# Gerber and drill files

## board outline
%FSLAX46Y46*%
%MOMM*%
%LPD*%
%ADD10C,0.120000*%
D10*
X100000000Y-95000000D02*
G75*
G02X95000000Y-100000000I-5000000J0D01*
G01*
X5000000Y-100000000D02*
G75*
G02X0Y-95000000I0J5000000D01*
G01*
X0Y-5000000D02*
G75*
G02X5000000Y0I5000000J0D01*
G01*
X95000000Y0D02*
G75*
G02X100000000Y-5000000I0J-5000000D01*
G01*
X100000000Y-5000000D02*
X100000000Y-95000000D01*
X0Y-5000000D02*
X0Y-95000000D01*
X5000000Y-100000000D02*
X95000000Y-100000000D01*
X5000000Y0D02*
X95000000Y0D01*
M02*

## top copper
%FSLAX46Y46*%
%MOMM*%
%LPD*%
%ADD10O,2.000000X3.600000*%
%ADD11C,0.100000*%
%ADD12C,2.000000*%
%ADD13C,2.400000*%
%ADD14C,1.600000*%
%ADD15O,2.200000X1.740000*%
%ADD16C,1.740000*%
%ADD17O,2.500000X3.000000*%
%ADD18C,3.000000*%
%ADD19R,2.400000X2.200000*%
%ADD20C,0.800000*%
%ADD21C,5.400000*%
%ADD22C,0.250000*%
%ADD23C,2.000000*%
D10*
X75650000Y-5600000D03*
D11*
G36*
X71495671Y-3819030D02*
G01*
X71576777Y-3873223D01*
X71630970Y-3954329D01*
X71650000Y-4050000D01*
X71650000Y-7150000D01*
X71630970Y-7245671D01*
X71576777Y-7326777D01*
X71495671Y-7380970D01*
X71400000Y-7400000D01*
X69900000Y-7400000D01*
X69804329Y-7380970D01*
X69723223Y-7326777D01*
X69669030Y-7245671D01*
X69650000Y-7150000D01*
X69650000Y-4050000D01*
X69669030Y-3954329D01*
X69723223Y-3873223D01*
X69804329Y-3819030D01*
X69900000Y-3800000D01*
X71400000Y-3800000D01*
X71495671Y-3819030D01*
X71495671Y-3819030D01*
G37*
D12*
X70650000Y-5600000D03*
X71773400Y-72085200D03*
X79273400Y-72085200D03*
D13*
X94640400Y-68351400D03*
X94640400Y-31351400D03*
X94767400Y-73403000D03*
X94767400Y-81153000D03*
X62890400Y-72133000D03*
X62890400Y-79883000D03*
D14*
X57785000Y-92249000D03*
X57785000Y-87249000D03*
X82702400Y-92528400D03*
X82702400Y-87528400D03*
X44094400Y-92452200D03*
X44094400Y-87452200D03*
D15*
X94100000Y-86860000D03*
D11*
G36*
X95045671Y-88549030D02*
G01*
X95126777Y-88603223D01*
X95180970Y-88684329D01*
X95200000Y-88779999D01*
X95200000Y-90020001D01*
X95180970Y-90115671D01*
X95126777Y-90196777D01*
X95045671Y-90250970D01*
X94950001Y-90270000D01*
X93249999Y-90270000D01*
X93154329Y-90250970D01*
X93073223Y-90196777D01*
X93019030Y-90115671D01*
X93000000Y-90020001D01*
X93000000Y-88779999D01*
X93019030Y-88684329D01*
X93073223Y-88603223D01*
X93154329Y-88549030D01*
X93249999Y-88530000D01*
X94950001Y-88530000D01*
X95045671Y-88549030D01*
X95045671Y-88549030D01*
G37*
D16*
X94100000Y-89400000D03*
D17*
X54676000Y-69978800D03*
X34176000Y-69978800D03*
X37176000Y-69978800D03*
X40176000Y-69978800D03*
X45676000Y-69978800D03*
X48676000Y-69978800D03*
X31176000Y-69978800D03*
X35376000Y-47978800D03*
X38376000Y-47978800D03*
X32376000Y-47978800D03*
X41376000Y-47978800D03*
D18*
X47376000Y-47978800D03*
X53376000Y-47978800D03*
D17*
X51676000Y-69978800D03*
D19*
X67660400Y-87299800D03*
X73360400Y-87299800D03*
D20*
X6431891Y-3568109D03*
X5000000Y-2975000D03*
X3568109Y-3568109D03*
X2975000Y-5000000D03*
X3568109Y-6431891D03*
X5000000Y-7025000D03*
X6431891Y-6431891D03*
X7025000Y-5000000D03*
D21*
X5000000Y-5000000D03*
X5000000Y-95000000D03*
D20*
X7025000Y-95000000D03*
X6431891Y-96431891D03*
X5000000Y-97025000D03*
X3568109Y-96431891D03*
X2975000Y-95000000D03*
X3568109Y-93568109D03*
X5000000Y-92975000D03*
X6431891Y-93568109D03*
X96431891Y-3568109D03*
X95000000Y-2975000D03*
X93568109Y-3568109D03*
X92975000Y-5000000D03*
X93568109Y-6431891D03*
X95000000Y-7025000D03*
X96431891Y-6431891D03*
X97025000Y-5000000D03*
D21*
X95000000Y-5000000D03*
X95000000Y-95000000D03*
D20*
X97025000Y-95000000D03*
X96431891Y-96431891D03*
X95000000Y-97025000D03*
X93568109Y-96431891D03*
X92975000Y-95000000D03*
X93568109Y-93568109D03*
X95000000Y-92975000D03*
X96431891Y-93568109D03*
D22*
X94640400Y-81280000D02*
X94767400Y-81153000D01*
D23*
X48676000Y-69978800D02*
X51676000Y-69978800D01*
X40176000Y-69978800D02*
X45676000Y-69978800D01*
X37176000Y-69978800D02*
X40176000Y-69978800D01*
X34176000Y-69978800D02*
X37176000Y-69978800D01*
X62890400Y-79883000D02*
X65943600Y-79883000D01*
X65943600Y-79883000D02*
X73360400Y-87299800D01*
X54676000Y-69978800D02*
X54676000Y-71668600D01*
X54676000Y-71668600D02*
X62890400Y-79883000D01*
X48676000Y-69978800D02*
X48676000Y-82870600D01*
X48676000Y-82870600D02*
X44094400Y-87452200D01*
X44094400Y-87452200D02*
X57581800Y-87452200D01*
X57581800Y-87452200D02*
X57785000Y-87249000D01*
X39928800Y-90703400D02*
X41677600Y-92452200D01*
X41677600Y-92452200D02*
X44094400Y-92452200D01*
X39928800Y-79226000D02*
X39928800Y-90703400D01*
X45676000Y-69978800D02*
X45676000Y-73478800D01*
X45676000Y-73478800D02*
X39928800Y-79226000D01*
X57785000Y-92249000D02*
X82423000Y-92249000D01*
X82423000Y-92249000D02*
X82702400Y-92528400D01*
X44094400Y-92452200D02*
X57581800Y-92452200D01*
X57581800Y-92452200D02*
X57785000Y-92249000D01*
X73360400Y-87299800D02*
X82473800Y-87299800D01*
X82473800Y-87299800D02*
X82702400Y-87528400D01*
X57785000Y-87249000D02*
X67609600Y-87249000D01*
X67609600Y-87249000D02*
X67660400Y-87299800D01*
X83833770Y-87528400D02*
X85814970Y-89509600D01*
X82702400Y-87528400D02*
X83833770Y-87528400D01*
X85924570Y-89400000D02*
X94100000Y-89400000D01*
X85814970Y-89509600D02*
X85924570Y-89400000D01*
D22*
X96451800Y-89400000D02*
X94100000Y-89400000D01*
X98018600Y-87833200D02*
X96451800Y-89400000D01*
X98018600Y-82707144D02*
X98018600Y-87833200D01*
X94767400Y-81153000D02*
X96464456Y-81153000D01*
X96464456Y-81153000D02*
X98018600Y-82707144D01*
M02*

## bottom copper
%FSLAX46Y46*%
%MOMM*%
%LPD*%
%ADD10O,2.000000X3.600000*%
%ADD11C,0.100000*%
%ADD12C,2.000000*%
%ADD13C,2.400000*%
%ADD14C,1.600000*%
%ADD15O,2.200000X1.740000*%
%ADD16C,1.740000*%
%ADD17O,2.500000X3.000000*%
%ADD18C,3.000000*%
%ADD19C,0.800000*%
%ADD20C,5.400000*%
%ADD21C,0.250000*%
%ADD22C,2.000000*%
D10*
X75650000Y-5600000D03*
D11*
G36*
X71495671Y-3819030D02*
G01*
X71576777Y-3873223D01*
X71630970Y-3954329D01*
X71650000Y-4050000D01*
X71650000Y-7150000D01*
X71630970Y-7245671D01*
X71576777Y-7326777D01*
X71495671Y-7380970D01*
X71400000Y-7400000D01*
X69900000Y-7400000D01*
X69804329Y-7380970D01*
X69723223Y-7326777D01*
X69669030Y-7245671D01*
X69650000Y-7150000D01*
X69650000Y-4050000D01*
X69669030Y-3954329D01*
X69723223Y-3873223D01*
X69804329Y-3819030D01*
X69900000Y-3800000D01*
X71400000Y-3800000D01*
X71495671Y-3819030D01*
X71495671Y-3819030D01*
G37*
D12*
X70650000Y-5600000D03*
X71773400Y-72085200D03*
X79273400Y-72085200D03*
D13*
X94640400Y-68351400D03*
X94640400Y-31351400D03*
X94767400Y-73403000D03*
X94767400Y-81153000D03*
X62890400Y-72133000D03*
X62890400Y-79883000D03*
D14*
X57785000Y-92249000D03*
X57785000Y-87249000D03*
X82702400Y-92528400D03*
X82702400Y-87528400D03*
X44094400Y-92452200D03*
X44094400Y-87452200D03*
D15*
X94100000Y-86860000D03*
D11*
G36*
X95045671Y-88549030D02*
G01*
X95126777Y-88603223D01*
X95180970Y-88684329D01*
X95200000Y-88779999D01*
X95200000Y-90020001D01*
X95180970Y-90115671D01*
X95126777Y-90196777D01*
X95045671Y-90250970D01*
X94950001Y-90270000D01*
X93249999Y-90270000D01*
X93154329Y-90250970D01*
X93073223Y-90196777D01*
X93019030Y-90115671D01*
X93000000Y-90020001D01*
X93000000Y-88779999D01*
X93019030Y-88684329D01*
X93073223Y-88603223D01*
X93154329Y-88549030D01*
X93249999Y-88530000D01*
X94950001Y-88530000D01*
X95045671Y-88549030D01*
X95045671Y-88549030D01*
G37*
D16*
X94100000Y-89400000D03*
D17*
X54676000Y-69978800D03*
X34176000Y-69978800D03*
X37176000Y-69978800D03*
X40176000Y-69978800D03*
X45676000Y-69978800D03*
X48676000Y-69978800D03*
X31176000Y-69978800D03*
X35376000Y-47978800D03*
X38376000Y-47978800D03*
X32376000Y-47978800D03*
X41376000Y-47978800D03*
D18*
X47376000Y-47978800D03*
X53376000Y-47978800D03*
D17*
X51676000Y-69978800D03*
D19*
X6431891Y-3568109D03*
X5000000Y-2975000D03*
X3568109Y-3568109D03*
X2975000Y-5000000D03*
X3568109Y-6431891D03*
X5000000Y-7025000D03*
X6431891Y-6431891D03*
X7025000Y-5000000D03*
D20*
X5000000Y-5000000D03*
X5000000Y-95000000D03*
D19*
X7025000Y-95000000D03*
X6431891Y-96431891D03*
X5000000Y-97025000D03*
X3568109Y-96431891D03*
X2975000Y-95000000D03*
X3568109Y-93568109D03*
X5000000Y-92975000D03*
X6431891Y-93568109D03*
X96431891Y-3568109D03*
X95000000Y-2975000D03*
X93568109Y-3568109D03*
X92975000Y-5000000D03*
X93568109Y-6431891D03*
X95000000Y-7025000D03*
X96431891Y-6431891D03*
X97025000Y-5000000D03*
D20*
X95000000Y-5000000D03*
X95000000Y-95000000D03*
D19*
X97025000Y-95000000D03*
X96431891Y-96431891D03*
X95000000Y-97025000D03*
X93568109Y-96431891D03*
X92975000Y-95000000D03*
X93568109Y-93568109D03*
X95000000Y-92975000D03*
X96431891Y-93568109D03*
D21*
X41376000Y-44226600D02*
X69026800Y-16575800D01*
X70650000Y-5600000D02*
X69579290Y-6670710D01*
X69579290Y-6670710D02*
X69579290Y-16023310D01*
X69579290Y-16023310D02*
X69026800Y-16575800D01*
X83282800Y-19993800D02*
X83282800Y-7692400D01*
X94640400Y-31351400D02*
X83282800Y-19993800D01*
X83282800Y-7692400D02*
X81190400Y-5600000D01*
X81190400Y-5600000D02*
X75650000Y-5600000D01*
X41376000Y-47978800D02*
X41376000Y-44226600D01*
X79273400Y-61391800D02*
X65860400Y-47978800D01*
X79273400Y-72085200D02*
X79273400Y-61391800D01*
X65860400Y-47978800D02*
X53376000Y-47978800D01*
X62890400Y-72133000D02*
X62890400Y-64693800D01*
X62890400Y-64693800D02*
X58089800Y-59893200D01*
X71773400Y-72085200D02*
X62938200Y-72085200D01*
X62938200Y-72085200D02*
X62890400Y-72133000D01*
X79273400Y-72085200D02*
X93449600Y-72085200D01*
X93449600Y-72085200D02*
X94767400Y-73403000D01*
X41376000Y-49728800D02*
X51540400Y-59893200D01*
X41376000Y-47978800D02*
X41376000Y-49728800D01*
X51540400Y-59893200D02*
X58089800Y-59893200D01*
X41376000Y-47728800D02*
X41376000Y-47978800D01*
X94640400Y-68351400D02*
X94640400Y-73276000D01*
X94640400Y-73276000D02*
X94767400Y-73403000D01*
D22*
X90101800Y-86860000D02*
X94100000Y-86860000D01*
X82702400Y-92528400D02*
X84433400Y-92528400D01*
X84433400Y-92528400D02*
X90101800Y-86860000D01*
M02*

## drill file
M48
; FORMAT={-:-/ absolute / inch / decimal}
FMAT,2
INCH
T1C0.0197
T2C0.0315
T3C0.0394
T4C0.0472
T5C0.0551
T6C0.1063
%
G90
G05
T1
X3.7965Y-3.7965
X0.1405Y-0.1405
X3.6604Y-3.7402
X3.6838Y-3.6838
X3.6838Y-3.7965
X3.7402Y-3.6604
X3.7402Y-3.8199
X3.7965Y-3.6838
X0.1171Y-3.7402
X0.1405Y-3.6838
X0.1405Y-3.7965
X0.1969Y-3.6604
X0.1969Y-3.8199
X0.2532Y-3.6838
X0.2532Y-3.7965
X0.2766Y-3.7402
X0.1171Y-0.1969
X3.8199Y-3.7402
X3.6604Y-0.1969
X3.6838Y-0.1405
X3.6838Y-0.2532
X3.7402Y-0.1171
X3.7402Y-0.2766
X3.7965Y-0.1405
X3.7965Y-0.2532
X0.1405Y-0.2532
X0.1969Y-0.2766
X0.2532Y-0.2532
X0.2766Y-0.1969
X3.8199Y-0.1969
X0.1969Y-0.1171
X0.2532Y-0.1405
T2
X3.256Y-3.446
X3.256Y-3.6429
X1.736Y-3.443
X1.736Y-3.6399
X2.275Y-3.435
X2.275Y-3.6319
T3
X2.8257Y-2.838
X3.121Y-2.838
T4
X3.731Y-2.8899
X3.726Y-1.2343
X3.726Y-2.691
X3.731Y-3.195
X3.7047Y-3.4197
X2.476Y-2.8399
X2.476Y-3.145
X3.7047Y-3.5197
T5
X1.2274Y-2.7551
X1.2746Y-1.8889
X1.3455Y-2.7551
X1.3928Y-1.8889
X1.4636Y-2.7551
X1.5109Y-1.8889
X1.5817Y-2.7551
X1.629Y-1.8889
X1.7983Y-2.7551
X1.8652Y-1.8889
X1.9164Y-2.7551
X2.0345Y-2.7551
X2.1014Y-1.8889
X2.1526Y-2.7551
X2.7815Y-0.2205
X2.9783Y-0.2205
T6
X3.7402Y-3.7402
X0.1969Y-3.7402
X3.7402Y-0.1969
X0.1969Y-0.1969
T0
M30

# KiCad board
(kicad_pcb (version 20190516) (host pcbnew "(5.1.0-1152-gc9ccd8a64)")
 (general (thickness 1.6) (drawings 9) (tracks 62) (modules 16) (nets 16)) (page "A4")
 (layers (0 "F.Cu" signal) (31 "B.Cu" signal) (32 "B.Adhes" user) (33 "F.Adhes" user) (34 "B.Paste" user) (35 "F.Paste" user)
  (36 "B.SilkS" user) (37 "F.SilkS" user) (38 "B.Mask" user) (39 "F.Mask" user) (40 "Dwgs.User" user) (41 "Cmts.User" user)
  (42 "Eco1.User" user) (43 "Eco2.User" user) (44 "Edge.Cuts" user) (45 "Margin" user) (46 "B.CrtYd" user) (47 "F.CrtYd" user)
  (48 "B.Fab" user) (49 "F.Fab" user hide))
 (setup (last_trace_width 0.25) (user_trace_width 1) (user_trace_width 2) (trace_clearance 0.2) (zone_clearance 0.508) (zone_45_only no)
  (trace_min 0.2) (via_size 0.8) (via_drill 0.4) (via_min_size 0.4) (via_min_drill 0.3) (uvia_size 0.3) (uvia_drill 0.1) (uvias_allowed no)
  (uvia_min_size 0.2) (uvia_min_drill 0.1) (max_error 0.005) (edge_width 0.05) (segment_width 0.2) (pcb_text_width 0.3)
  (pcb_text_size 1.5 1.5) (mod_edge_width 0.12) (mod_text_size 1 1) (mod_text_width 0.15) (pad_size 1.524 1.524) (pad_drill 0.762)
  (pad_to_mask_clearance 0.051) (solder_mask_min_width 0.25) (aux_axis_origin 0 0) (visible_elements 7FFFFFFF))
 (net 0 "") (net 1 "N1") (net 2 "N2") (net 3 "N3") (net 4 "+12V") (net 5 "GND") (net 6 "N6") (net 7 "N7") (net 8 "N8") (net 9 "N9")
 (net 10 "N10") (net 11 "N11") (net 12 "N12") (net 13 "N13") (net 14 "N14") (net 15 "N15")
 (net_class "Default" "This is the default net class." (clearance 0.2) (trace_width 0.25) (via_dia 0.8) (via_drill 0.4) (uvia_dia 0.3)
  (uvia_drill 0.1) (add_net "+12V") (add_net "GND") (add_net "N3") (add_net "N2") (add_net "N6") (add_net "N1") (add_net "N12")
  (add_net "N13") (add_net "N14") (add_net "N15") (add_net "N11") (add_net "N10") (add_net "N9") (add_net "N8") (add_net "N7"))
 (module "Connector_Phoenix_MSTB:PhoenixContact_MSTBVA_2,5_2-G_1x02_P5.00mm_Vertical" (layer "F.Cu") (at 70.65 5.6)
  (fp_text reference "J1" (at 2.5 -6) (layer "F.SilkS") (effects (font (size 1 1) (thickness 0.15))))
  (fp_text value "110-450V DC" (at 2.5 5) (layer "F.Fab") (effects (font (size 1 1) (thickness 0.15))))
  (pad "2" thru_hole oval (at 5 0) (size 2 3.6) (drill 1.4) (layers *.Cu *.Mask) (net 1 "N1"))
  (pad "1" thru_hole roundrect (at 0 0) (size 2 3.6) (drill 1.4) (layers *.Cu *.Mask) (roundrect_rratio 0.125) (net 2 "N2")))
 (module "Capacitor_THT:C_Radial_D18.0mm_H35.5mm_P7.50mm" (layer "F.Cu") (at 79.2734 72.0852 180)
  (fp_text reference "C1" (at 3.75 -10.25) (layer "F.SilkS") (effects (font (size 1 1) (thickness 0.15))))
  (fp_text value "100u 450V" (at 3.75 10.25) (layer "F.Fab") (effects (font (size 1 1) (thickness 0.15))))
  (pad "2" thru_hole circle (at 7.5 0 180) (size 2 2) (drill 1) (layers *.Cu *.Mask) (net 2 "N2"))
  (pad "1" thru_hole circle (at 0 0 180) (size 2 2) (drill 1) (layers *.Cu *.Mask) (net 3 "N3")))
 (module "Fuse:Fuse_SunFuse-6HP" (layer "F.Cu") (at 94.6404 68.3514 90)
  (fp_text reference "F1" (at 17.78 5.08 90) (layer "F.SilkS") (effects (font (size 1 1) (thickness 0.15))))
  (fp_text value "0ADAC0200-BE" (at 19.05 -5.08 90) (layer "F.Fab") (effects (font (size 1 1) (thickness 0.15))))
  (pad "1" thru_hole circle (at 0 0 90) (size 2.4 2.4) (drill 1.2) (layers *.Cu *.Mask) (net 3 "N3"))
  (pad "2" thru_hole circle (at 37 0 90) (size 2.4 2.4) (drill 1.2) (layers *.Cu *.Mask) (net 1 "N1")))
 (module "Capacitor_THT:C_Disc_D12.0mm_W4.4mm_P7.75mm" (layer "F.Cu") (at 94.7674 81.153 90)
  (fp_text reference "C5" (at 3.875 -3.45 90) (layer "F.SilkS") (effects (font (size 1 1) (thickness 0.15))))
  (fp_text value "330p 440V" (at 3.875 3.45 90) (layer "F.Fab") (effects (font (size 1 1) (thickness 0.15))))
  (pad "2" thru_hole circle (at 7.75 0 90) (size 2.4 2.4) (drill 1.2) (layers *.Cu *.Mask) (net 3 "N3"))
  (pad "1" thru_hole circle (at 0 0 90) (size 2.4 2.4) (drill 1.2) (layers *.Cu *.Mask) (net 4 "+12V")))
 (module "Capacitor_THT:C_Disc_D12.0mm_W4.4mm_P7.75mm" (layer "F.Cu") (at 62.8904 79.883 90)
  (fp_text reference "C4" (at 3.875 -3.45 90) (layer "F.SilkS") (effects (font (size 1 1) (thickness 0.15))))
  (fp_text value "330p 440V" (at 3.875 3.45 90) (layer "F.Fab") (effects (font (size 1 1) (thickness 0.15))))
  (pad "2" thru_hole circle (at 7.75 0 90) (size 2.4 2.4) (drill 1.2) (layers *.Cu *.Mask) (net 2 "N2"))
  (pad "1" thru_hole circle (at 0 0 90) (size 2.4 2.4) (drill 1.2) (layers *.Cu *.Mask) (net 4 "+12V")))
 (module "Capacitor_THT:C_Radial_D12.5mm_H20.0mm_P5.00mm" (layer "F.Cu") (at 57.785 87.249 270)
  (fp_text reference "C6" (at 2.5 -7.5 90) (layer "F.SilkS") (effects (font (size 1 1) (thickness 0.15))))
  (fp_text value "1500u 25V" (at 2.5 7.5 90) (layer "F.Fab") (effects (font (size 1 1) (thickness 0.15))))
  (pad "2" thru_hole circle (at 5 0 270) (size 1.6 1.6) (drill 0.8) (layers *.Cu *.Mask) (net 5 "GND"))
  (pad "1" thru_hole circle (at 0 0 270) (size 1.6 1.6) (drill 0.8) (layers *.Cu *.Mask) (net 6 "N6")))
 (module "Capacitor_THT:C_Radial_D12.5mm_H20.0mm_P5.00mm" (layer "F.Cu") (at 82.7024 87.5284 270)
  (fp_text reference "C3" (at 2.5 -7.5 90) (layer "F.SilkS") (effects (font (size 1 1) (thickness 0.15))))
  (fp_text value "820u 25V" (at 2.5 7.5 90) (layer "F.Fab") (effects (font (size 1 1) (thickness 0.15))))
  (pad "2" thru_hole circle (at 5 0 270) (size 1.6 1.6) (drill 0.8) (layers *.Cu *.Mask) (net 5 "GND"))
  (pad "1" thru_hole circle (at 0 0 270) (size 1.6 1.6) (drill 0.8) (layers *.Cu *.Mask) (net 4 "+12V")))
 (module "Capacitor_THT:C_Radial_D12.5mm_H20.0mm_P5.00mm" (layer "F.Cu") (at 44.0944 87.4522 270)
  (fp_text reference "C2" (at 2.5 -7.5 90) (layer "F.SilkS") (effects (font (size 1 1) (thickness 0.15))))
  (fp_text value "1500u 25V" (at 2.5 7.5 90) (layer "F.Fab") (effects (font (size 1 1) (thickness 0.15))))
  (pad "2" thru_hole circle (at 5 0 270) (size 1.6 1.6) (drill 0.8) (layers *.Cu *.Mask) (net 5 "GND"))
  (pad "1" thru_hole circle (at 0 0 270) (size 1.6 1.6) (drill 0.8) (layers *.Cu *.Mask) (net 6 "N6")))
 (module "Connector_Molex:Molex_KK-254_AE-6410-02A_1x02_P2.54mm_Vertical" (layer "F.Cu") (at 94.1 89.4 90)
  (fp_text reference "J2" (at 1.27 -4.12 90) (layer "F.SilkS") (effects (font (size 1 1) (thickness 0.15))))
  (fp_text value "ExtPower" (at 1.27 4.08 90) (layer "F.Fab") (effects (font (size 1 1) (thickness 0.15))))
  (pad "2" thru_hole oval (at 2.54 0 90) (size 1.74 2.2) (drill 1.2) (layers *.Cu *.Mask) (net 5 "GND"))
  (pad "1" thru_hole roundrect (at 0 0 90) (size 1.74 2.2) (drill 1.2) (layers *.Cu *.Mask) (roundrect_rratio 0.143678) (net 4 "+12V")))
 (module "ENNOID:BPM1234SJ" (layer "F.Cu") (at 42.926 58.9788 270)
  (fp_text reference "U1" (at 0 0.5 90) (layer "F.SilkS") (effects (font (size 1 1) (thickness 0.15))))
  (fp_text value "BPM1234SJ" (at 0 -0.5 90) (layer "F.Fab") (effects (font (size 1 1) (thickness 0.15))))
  (pad "14" thru_hole oval (at 11 -11.75) (size 2.5 3) (drill 1.4) (layers *.Cu *.Mask) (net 4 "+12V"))
  (pad "8" thru_hole oval (at 11 8.75) (size 2.5 3) (drill 1.4) (layers *.Cu *.Mask) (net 5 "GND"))
  (pad "9" thru_hole oval (at 11 5.75) (size 2.5 3) (drill 1.4) (layers *.Cu *.Mask) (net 5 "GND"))
  (pad "10" thru_hole oval (at 11 2.75) (size 2.5 3) (drill 1.4) (layers *.Cu *.Mask) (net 5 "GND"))
  (pad "11" thru_hole oval (at 11 -2.75) (size 2.5 3) (drill 1.4) (layers *.Cu *.Mask) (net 5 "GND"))
  (pad "12" thru_hole oval (at 11 -5.75) (size 2.5 3) (drill 1.4) (layers *.Cu *.Mask) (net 6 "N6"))
  (pad "7" thru_hole oval (at 11 11.75 180) (size 2.5 3) (drill 1.4) (layers *.Cu *.Mask) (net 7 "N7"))
  (pad "6" thru_hole oval (at -11 7.55) (size 2.5 3) (drill 1.4) (layers *.Cu *.Mask) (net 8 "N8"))
  (pad "5" thru_hole oval (at -11 4.55) (size 2.5 3) (drill 1.4) (layers *.Cu *.Mask) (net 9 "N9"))
  (pad "4" thru_hole oval (at -11 10.55) (size 2.5 3) (drill 1.4) (layers *.Cu *.Mask) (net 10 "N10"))
  (pad "3" thru_hole oval (at -11 1.55) (size 2.5 3) (drill 1.4) (layers *.Cu *.Mask) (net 2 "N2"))
  (pad "2" thru_hole circle (at -11 -4.45) (size 3 3) (drill 1.4) (layers *.Cu *.Mask) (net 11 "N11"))
  (pad "1" thru_hole circle (at -11 -10.45) (size 3 3) (drill 1.4) (layers *.Cu *.Mask) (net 3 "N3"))
  (pad "13" thru_hole oval (at 11 -8.75) (size 2.5 3) (drill 1.4) (layers *.Cu *.Mask) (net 6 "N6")))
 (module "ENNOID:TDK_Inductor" (layer "F.Cu") (at 70.5104 87.2998)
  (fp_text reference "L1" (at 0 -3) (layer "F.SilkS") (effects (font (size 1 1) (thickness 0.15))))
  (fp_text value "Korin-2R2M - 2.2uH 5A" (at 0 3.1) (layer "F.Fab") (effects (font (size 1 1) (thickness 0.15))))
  (pad "1" smd rect (at -2.85 0) (size 2.4 2.2) (layers "F.Cu" "F.Paste" "F.Mask") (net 6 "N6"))
  (pad "2" smd rect (at 2.85 0) (size 2.4 2.2) (layers "F.Cu" "F.Paste" "F.Mask") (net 4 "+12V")))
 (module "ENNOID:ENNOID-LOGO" (layer "F.Cu") (at 15.3924 51.8922 270)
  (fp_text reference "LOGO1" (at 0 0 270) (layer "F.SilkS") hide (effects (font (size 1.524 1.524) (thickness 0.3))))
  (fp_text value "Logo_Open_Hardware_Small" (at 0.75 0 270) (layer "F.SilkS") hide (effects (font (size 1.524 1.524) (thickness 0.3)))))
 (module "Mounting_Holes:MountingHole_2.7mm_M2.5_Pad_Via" (layer "F.Cu") (at 5 5)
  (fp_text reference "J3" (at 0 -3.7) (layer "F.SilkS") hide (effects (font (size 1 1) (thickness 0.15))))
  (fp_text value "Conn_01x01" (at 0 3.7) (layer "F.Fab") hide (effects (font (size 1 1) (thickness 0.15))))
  (pad "1" thru_hole circle (at 1.431891 -1.431891) (size 0.8 0.8) (drill 0.5) (layers *.Cu *.Mask) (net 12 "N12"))
  (pad "1" thru_hole circle (at 0 -2.025) (size 0.8 0.8) (drill 0.5) (layers *.Cu *.Mask) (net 12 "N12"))
  (pad "1" thru_hole circle (at -1.431891 -1.431891) (size 0.8 0.8) (drill 0.5) (layers *.Cu *.Mask) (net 12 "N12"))
  (pad "1" thru_hole circle (at -2.025 0) (size 0.8 0.8) (drill 0.5) (layers *.Cu *.Mask) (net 12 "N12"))
  (pad "1" thru_hole circle (at -1.431891 1.431891) (size 0.8 0.8) (drill 0.5) (layers *.Cu *.Mask) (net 12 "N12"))
  (pad "1" thru_hole circle (at 0 2.025) (size 0.8 0.8) (drill 0.5) (layers *.Cu *.Mask) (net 12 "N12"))
  (pad "1" thru_hole circle (at 1.431891 1.431891) (size 0.8 0.8) (drill 0.5) (layers *.Cu *.Mask) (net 12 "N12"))
  (pad "1" thru_hole circle (at 2.025 0) (size 0.8 0.8) (drill 0.5) (layers *.Cu *.Mask) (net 12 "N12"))
  (pad "1" thru_hole circle (at 0 0) (size 5.4 5.4) (drill 2.7) (layers *.Cu *.Mask) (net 12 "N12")))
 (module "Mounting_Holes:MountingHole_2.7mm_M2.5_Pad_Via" (layer "F.Cu") (at 5 95)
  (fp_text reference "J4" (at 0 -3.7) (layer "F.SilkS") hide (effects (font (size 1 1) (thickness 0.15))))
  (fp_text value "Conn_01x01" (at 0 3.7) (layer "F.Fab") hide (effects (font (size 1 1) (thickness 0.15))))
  (pad "1" thru_hole circle (at 0 0) (size 5.4 5.4) (drill 2.7) (layers *.Cu *.Mask) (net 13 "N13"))
  (pad "1" thru_hole circle (at 2.025 0) (size 0.8 0.8) (drill 0.5) (layers *.Cu *.Mask) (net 13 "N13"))
  (pad "1" thru_hole circle (at 1.431891 1.431891) (size 0.8 0.8) (drill 0.5) (layers *.Cu *.Mask) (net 13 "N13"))
  (pad "1" thru_hole circle (at 0 2.025) (size 0.8 0.8) (drill 0.5) (layers *.Cu *.Mask) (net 13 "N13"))
  (pad "1" thru_hole circle (at -1.431891 1.431891) (size 0.8 0.8) (drill 0.5) (layers *.Cu *.Mask) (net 13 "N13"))
  (pad "1" thru_hole circle (at -2.025 0) (size 0.8 0.8) (drill 0.5) (layers *.Cu *.Mask) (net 13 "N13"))
  (pad "1" thru_hole circle (at -1.431891 -1.431891) (size 0.8 0.8) (drill 0.5) (layers *.Cu *.Mask) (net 13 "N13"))
  (pad "1" thru_hole circle (at 0 -2.025) (size 0.8 0.8) (drill 0.5) (layers *.Cu *.Mask) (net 13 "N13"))
  (pad "1" thru_hole circle (at 1.431891 -1.431891) (size 0.8 0.8) (drill 0.5) (layers *.Cu *.Mask) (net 13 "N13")))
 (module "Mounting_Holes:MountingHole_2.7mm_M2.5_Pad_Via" (layer "F.Cu") (at 95 5)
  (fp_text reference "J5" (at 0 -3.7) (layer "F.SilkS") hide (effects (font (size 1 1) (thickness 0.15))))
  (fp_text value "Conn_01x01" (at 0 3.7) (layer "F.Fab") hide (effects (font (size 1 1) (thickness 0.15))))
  (pad "1" thru_hole circle (at 1.431891 -1.431891) (size 0.8 0.8) (drill 0.5) (layers *.Cu *.Mask) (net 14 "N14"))
  (pad "1" thru_hole circle (at 0 -2.025) (size 0.8 0.8) (drill 0.5) (layers *.Cu *.Mask) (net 14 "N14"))
  (pad "1" thru_hole circle (at -1.431891 -1.431891) (size 0.8 0.8) (drill 0.5) (layers *.Cu *.Mask) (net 14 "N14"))
  (pad "1" thru_hole circle (at -2.025 0) (size 0.8 0.8) (drill 0.5) (layers *.Cu *.Mask) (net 14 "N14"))
  (pad "1" thru_hole circle (at -1.431891 1.431891) (size 0.8 0.8) (drill 0.5) (layers *.Cu *.Mask) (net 14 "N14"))
  (pad "1" thru_hole circle (at 0 2.025) (size 0.8 0.8) (drill 0.5) (layers *.Cu *.Mask) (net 14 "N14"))
  (pad "1" thru_hole circle (at 1.431891 1.431891) (size 0.8 0.8) (drill 0.5) (layers *.Cu *.Mask) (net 14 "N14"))
  (pad "1" thru_hole circle (at 2.025 0) (size 0.8 0.8) (drill 0.5) (layers *.Cu *.Mask) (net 14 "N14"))
  (pad "1" thru_hole circle (at 0 0) (size 5.4 5.4) (drill 2.7) (layers *.Cu *.Mask) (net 14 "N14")))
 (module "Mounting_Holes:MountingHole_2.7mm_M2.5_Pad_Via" (layer "F.Cu") (at 95 95)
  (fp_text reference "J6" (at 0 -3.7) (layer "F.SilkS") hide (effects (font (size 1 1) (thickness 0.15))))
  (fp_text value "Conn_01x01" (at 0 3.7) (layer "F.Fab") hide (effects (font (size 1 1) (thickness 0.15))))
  (pad "1" thru_hole circle (at 0 0) (size 5.4 5.4) (drill 2.7) (layers *.Cu *.Mask) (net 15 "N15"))
  (pad "1" thru_hole circle (at 2.025 0) (size 0.8 0.8) (drill 0.5) (layers *.Cu *.Mask) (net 15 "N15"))
  (pad "1" thru_hole circle (at 1.431891 1.431891) (size 0.8 0.8) (drill 0.5) (layers *.Cu *.Mask) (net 15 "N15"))
  (pad "1" thru_hole circle (at 0 2.025) (size 0.8 0.8) (drill 0.5) (layers *.Cu *.Mask) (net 15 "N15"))
  (pad "1" thru_hole circle (at -1.431891 1.431891) (size 0.8 0.8) (drill 0.5) (layers *.Cu *.Mask) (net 15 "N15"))
  (pad "1" thru_hole circle (at -2.025 0) (size 0.8 0.8) (drill 0.5) (layers *.Cu *.Mask) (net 15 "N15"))
  (pad "1" thru_hole circle (at -1.431891 -1.431891) (size 0.8 0.8) (drill 0.5) (layers *.Cu *.Mask) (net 15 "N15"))
  (pad "1" thru_hole circle (at 0 -2.025) (size 0.8 0.8) (drill 0.5) (layers *.Cu *.Mask) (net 15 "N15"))
  (pad "1" thru_hole circle (at 1.431891 -1.431891) (size 0.8 0.8) (drill 0.5) (layers *.Cu *.Mask) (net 15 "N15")))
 (gr_arc (start 95 95) (end 95 100) (angle -90) (layer "Edge.Cuts") (width 0.12))
 (gr_arc (start 5 95) (end 0 95) (angle -90) (layer "Edge.Cuts") (width 0.12))
 (gr_arc (start 5 5) (end 5 0) (angle -90) (layer "Edge.Cuts") (width 0.12))
 (gr_arc (start 95 5) (end 100 5) (angle -90) (layer "Edge.Cuts") (width 0.12))
 (gr_line (start 100 5) (end 100 95) (layer "Edge.Cuts") (width 0.12))
 (gr_line (start 0 5) (end 0 95) (layer "Edge.Cuts") (width 0.12))
 (gr_line (start 5 100) (end 95 100) (layer "Edge.Cuts") (width 0.12))
 (gr_line (start 5 0) (end 95 0) (layer "Edge.Cuts") (width 0.12))
 (segment (start 41.376 44.2266) (end 69.0268 16.5758) (width 0.25) (layer "B.Cu") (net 2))
 (segment (start 70.65 5.6) (end 69.57929 6.67071) (width 0.25) (layer "B.Cu") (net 2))
 (segment (start 69.57929 6.67071) (end 69.57929 16.02331) (width 0.25) (layer "B.Cu") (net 2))
 (segment (start 69.57929 16.02331) (end 69.0268 16.5758) (width 0.25) (layer "B.Cu") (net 2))
 (segment (start 83.2828 19.9938) (end 83.2828 7.6924) (width 0.25) (layer "B.Cu") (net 1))
 (segment (start 94.6404 31.3514) (end 83.2828 19.9938) (width 0.25) (layer "B.Cu") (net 1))
 (segment (start 83.2828 7.6924) (end 81.1904 5.6) (width 0.25) (layer "B.Cu") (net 1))
 (segment (start 81.1904 5.6) (end 75.65 5.6) (width 0.25) (layer "B.Cu") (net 1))
 (segment (start 94.6404 81.28) (end 94.7674 81.153) (width 0.25) (layer "F.Cu") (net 4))
 (segment (start 48.676 69.9788) (end 51.676 69.9788) (width 2) (layer "F.Cu") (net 6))
 (segment (start 40.176 69.9788) (end 45.676 69.9788) (width 2) (layer "F.Cu") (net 5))
 (segment (start 37.176 69.9788) (end 40.176 69.9788) (width 2) (layer "F.Cu") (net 5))
 (segment (start 34.176 69.9788) (end 37.176 69.9788) (width 2) (layer "F.Cu") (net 5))
 (segment (start 62.8904 79.883) (end 65.9436 79.883) (width 2) (layer "F.Cu") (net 4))
 (segment (start 65.9436 79.883) (end 73.3604 87.2998) (width 2) (layer "F.Cu") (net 4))
 (segment (start 54.676 69.9788) (end 54.676 71.6686) (width 2) (layer "F.Cu") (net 4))
 (segment (start 54.676 71.6686) (end 62.8904 79.883) (width 2) (layer "F.Cu") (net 4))
 (segment (start 41.376 47.9788) (end 41.376 44.2266) (width 0.25) (layer "B.Cu") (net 2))
 (segment (start 79.2734 61.3918) (end 65.8604 47.9788) (width 0.25) (layer "B.Cu") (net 3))
 (segment (start 79.2734 72.0852) (end 79.2734 61.3918) (width 0.25) (layer "B.Cu") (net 3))
 (segment (start 65.8604 47.9788) (end 53.376 47.9788) (width 0.25) (layer "B.Cu") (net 3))
 (segment (start 62.8904 72.133) (end 62.8904 64.6938) (width 0.25) (layer "B.Cu") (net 2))
 (segment (start 62.8904 64.6938) (end 58.0898 59.8932) (width 0.25) (layer "B.Cu") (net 2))
 (segment (start 71.7734 72.0852) (end 62.9382 72.0852) (width 0.25) (layer "B.Cu") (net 2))
 (segment (start 62.9382 72.0852) (end 62.8904 72.133) (width 0.25) (layer "B.Cu") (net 2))
 (segment (start 79.2734 72.0852) (end 93.4496 72.0852) (width 0.25) (layer "B.Cu") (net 3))
 (segment (start 93.4496 72.0852) (end 94.7674 73.403) (width 0.25) (layer "B.Cu") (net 3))
 (segment (start 48.676 69.9788) (end 48.676 82.8706) (width 2) (layer "F.Cu") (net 6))
 (segment (start 48.676 82.8706) (end 44.0944 87.4522) (width 2) (layer "F.Cu") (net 6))
 (segment (start 44.0944 87.4522) (end 57.5818 87.4522) (width 2) (layer "F.Cu") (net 6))
 (segment (start 57.5818 87.4522) (end 57.785 87.249) (width 2) (layer "F.Cu") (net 6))
 (segment (start 39.9288 90.7034) (end 41.6776 92.4522) (width 2) (layer "F.Cu") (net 5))
 (segment (start 41.6776 92.4522) (end 44.0944 92.4522) (width 2) (layer "F.Cu") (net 5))
 (segment (start 39.9288 79.226) (end 39.9288 90.7034) (width 2) (layer "F.Cu") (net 5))
 (segment (start 45.676 69.9788) (end 45.676 73.4788) (width 2) (layer "F.Cu") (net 5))
 (segment (start 45.676 73.4788) (end 39.9288 79.226) (width 2) (layer "F.Cu") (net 5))
 (segment (start 57.785 92.249) (end 82.423 92.249) (width 2) (layer "F.Cu") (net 5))
 (segment (start 82.423 92.249) (end 82.7024 92.5284) (width 2) (layer "F.Cu") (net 5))
 (segment (start 44.0944 92.4522) (end 57.5818 92.4522) (width 2) (layer "F.Cu") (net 5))
 (segment (start 57.5818 92.4522) (end 57.785 92.249) (width 2) (layer "F.Cu") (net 5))
 (segment (start 73.3604 87.2998) (end 82.4738 87.2998) (width 2) (layer "F.Cu") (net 4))
 (segment (start 82.4738 87.2998) (end 82.7024 87.5284) (width 2) (layer "F.Cu") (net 4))
 (segment (start 57.785 87.249) (end 67.6096 87.249) (width 2) (layer "F.Cu") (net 6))
 (segment (start 67.6096 87.249) (end 67.6604 87.2998) (width 2) (layer "F.Cu") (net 6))
 (segment (start 41.376 49.7288) (end 51.5404 59.8932) (width 0.25) (layer "B.Cu") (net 2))
 (segment (start 41.376 47.9788) (end 41.376 49.7288) (width 0.25) (layer "B.Cu") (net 2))
 (segment (start 51.5404 59.8932) (end 58.0898 59.8932) (width 0.25) (layer "B.Cu") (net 2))
 (segment (start 41.376 47.7288) (end 41.376 47.9788) (width 0.25) (layer "B.Cu") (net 2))
 (segment (start 94.6404 68.3514) (end 94.6404 73.276) (width 0.25) (layer "B.Cu") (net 3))
 (segment (start 94.6404 73.276) (end 94.7674 73.403) (width 0.25) (layer "B.Cu") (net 3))
 (segment (start 83.83377 87.5284) (end 85.81497 89.5096) (width 2) (layer "F.Cu") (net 4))
 (segment (start 82.7024 87.5284) (end 83.83377 87.5284) (width 2) (layer "F.Cu") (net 4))
 (segment (start 85.92457 89.4) (end 94.1 89.4) (width 2) (layer "F.Cu") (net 4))
 (segment (start 85.81497 89.5096) (end 85.92457 89.4) (width 2) (layer "F.Cu") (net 4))
 (segment (start 90.1018 86.86) (end 94.1 86.86) (width 2) (layer "B.Cu") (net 5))
 (segment (start 82.7024 92.5284) (end 84.4334 92.5284) (width 2) (layer "B.Cu") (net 5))
 (segment (start 84.4334 92.5284) (end 90.1018 86.86) (width 2) (layer "B.Cu") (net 5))
 (segment (start 96.4518 89.4) (end 94.1 89.4) (width 0.25) (layer "F.Cu") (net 4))
 (segment (start 98.0186 87.8332) (end 96.4518 89.4) (width 0.25) (layer "F.Cu") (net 4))
 (segment (start 98.0186 82.707144) (end 98.0186 87.8332) (width 0.25) (layer "F.Cu") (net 4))
 (segment (start 94.7674 81.153) (end 96.464456 81.153) (width 0.25) (layer "F.Cu") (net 4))
 (segment (start 96.464456 81.153) (end 98.0186 82.707144) (width 0.25) (layer "F.Cu") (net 4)))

